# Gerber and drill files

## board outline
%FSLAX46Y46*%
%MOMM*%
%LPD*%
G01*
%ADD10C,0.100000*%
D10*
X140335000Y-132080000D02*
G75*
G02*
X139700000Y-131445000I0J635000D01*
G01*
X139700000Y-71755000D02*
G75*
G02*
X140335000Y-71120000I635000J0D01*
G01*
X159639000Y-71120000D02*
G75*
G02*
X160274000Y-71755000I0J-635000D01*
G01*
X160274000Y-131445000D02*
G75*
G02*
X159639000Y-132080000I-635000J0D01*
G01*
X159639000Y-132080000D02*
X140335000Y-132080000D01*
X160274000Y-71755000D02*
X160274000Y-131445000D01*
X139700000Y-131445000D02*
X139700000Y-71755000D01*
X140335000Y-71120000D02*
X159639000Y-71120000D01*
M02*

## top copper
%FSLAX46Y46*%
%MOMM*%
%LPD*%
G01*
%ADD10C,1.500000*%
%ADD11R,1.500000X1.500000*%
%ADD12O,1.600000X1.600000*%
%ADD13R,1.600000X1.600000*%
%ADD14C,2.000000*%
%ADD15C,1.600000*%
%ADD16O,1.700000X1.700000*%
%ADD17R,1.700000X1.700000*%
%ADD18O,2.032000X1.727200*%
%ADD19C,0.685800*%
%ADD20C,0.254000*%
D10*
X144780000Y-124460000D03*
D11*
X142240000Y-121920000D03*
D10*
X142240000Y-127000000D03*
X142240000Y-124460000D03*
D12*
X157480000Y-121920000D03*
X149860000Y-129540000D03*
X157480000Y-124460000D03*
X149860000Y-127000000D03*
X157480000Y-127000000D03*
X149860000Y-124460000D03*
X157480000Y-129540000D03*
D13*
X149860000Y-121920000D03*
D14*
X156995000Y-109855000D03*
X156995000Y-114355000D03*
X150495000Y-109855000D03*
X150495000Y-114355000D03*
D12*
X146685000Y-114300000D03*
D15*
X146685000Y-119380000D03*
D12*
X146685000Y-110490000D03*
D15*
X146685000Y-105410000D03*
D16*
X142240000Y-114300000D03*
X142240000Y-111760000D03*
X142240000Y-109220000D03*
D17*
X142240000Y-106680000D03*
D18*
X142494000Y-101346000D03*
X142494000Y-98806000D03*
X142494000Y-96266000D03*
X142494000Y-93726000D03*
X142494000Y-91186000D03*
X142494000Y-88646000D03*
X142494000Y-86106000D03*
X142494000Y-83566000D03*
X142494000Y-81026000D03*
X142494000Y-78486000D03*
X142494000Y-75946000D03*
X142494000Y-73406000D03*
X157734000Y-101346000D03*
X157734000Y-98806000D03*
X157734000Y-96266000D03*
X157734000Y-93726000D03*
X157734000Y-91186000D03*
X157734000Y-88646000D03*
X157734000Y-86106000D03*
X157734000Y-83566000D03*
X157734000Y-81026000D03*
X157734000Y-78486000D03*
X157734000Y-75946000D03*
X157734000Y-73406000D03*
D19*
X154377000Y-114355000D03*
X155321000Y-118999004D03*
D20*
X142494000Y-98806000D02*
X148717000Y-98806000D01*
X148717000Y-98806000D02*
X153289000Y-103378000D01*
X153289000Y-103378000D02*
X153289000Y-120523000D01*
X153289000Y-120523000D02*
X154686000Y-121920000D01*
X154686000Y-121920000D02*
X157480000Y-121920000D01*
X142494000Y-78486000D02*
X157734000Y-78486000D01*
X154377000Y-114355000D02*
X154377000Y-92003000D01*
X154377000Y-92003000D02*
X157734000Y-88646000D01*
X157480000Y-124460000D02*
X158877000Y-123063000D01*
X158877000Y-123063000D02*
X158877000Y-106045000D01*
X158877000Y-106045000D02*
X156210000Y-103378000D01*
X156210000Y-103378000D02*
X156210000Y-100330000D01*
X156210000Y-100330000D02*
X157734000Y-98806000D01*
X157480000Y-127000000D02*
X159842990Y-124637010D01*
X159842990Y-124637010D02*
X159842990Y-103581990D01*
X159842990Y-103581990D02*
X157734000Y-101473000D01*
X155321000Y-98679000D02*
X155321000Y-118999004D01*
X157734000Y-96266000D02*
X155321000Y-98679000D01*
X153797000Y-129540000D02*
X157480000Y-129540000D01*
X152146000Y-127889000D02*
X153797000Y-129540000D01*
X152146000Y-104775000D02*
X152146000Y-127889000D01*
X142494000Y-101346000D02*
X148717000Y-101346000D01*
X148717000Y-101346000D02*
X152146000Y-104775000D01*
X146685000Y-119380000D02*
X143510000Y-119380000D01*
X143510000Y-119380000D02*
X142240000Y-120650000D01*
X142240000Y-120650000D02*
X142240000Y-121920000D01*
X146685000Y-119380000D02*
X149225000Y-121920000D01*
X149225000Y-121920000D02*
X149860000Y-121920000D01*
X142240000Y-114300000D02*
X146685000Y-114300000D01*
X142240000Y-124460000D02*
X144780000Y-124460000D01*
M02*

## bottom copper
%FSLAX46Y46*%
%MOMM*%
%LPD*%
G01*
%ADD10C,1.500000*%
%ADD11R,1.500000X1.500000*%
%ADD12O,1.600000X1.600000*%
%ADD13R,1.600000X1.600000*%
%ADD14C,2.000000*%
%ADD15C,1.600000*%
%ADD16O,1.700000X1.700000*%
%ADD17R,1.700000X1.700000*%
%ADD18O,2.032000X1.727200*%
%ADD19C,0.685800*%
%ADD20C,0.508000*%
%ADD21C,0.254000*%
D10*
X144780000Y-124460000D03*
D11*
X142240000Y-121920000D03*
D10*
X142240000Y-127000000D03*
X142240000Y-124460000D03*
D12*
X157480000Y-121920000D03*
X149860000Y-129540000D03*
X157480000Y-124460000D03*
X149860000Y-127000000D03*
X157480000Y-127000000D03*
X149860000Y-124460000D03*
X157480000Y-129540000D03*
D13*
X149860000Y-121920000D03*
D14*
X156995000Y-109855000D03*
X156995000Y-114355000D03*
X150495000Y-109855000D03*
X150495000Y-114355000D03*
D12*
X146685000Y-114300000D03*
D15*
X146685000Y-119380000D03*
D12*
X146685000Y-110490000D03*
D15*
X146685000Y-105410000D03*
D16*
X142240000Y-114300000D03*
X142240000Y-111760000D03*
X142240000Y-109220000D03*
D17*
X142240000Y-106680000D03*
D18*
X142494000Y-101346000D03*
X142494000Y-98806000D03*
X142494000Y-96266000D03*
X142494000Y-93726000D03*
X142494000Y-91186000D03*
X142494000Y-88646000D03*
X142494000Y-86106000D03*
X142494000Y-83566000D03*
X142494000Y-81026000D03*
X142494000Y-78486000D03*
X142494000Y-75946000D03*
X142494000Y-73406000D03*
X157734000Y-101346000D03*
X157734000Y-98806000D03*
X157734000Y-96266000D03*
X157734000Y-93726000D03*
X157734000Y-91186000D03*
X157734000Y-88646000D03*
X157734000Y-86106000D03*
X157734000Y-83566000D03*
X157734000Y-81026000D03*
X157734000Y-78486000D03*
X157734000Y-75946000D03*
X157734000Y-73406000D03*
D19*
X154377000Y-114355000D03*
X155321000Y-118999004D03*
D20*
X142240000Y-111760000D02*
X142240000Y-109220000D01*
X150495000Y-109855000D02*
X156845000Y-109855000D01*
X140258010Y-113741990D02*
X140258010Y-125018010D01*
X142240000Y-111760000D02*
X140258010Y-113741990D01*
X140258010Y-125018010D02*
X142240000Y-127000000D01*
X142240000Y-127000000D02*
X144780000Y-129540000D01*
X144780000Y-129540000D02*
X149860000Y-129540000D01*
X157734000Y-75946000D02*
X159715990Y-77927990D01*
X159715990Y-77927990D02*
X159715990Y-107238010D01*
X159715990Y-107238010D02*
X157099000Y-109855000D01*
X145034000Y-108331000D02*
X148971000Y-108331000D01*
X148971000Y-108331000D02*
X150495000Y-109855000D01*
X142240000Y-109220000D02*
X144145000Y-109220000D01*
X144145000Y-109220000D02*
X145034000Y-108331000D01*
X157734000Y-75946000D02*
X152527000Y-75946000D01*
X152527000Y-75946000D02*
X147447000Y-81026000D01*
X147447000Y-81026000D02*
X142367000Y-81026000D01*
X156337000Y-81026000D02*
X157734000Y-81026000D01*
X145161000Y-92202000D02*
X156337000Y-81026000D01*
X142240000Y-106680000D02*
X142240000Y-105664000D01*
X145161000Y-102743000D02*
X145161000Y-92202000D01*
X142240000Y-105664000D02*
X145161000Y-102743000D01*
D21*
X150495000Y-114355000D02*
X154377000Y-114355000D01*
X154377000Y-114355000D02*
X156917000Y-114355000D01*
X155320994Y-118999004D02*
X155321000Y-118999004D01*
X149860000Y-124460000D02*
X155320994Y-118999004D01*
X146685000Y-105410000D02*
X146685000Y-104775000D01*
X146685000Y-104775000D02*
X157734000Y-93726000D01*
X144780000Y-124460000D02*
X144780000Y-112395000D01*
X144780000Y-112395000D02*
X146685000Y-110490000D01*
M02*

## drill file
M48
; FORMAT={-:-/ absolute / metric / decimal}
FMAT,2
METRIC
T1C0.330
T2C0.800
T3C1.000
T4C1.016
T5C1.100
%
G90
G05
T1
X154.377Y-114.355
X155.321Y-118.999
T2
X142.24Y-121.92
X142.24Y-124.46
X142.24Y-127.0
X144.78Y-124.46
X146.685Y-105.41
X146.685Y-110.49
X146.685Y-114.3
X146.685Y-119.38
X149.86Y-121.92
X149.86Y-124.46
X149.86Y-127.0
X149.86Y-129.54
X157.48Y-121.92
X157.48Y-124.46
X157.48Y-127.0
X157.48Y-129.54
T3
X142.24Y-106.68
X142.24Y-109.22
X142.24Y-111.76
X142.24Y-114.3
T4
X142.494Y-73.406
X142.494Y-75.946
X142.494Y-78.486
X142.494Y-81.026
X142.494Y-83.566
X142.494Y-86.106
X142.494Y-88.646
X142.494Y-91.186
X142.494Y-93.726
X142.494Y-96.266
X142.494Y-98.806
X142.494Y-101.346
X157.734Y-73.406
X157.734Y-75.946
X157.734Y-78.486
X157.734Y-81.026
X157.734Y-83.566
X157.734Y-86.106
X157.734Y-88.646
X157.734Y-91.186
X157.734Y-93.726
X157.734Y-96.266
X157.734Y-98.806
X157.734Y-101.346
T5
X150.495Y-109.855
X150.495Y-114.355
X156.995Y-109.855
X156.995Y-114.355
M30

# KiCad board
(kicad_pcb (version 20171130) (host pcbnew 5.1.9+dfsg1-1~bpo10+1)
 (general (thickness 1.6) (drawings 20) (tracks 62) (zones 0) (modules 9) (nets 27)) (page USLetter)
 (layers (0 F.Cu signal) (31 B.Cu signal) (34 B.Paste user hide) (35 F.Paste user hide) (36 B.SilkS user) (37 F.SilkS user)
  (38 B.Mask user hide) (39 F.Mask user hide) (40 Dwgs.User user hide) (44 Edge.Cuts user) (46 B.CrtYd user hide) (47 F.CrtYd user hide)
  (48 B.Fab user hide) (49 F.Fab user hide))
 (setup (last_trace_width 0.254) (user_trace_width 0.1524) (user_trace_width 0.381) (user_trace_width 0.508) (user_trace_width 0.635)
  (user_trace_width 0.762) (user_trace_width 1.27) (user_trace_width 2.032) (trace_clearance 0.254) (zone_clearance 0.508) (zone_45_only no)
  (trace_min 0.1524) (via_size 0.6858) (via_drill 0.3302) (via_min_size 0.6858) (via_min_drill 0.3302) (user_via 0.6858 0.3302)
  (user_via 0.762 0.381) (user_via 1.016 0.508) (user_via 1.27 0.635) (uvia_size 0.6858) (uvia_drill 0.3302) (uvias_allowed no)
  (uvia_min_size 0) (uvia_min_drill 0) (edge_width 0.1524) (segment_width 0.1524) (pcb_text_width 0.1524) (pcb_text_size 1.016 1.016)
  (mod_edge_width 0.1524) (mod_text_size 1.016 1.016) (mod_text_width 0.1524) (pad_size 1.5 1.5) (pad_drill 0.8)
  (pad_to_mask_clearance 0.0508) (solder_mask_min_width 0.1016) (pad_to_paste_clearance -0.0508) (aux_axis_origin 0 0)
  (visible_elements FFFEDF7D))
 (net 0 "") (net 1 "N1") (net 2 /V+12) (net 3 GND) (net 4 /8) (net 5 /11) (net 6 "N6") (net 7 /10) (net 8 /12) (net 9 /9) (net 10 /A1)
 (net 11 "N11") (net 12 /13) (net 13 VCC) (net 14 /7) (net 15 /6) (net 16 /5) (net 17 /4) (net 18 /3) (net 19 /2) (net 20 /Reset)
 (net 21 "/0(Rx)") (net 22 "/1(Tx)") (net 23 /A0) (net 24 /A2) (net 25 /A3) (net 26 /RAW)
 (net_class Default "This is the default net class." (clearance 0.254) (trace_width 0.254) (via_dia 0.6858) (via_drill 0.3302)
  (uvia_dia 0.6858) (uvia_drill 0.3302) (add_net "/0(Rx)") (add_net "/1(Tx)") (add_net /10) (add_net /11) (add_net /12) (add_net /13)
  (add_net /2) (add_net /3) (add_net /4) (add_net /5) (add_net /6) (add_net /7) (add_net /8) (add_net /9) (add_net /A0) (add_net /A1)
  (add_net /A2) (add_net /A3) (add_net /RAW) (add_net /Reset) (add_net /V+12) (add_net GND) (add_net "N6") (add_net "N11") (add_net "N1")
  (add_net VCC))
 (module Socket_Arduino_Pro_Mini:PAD (layer F.Cu) (at 144.78 124.46)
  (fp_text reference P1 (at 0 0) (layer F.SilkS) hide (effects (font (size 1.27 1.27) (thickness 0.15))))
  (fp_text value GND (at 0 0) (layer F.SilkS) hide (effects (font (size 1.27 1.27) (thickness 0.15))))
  (pad 1 thru_hole circle (at 0 0) (size 1.5 1.5) (drill 0.8) (layers *.Cu *.Mask) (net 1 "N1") (solder_mask_margin 0.0762)))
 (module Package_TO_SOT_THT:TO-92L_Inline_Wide (layer F.Cu) (at 142.24 121.92 270)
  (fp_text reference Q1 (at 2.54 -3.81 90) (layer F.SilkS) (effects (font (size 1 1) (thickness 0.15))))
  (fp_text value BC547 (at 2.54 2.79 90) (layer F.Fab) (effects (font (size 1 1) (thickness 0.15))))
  (pad 1 thru_hole rect (at 0 0 270) (size 1.5 1.5) (drill 0.8) (layers *.Cu *.Mask) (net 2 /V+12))
  (pad 3 thru_hole circle (at 5.08 0 270) (size 1.5 1.5) (drill 0.8) (layers *.Cu *.Mask) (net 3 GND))
  (pad 2 thru_hole circle (at 2.54 0 270) (size 1.5 1.5) (drill 0.8) (layers *.Cu *.Mask) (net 1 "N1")))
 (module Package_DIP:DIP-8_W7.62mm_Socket (layer F.Cu) (at 149.86 121.92)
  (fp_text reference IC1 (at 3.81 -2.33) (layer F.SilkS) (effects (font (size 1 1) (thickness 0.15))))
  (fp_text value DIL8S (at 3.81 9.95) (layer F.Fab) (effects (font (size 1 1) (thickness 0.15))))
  (pad 8 thru_hole oval (at 7.62 0) (size 1.6 1.6) (drill 0.8) (layers *.Cu *.Mask) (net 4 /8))
  (pad 4 thru_hole oval (at 0 7.62) (size 1.6 1.6) (drill 0.8) (layers *.Cu *.Mask) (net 3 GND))
  (pad 7 thru_hole oval (at 7.62 2.54) (size 1.6 1.6) (drill 0.8) (layers *.Cu *.Mask) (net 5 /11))
  (pad 3 thru_hole oval (at 0 5.08) (size 1.6 1.6) (drill 0.8) (layers *.Cu *.Mask) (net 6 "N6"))
  (pad 6 thru_hole oval (at 7.62 5.08) (size 1.6 1.6) (drill 0.8) (layers *.Cu *.Mask) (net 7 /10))
  (pad 2 thru_hole oval (at 0 2.54) (size 1.6 1.6) (drill 0.8) (layers *.Cu *.Mask) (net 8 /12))
  (pad 5 thru_hole oval (at 7.62 7.62) (size 1.6 1.6) (drill 0.8) (layers *.Cu *.Mask) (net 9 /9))
  (pad 1 thru_hole rect (at 0 0) (size 1.6 1.6) (drill 0.8) (layers *.Cu *.Mask) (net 2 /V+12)))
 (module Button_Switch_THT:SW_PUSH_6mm (layer F.Cu) (at 150.495 109.855)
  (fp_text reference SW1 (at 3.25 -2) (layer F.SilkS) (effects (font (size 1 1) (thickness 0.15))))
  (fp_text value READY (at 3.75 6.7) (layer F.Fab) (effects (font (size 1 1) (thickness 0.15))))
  (pad 1 thru_hole circle (at 6.5 0 90) (size 2 2) (drill 1.1) (layers *.Cu *.Mask) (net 3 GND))
  (pad 2 thru_hole circle (at 6.5 4.5 90) (size 2 2) (drill 1.1) (layers *.Cu *.Mask) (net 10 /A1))
  (pad 1 thru_hole circle (at 0 0 90) (size 2 2) (drill 1.1) (layers *.Cu *.Mask) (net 3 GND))
  (pad 2 thru_hole circle (at 0 4.5 90) (size 2 2) (drill 1.1) (layers *.Cu *.Mask) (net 10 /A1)))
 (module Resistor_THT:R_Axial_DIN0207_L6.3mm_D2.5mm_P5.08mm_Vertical (layer F.Cu) (at 146.685 119.38 90)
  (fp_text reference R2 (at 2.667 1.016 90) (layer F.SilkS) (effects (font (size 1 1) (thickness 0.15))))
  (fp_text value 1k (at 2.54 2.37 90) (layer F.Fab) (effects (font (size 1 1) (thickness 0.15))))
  (pad 2 thru_hole oval (at 5.08 0 90) (size 1.6 1.6) (drill 0.8) (layers *.Cu *.Mask) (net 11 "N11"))
  (pad 1 thru_hole circle (at 0 0 90) (size 1.6 1.6) (drill 0.8) (layers *.Cu *.Mask) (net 2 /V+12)))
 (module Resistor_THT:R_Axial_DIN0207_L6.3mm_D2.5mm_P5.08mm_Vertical (layer F.Cu) (at 146.685 105.41 270)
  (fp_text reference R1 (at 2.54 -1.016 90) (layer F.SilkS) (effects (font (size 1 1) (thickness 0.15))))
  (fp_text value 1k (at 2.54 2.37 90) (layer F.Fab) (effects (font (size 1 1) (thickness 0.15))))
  (pad 2 thru_hole oval (at 5.08 0 270) (size 1.6 1.6) (drill 0.8) (layers *.Cu *.Mask) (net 1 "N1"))
  (pad 1 thru_hole circle (at 0 0 270) (size 1.6 1.6) (drill 0.8) (layers *.Cu *.Mask) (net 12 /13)))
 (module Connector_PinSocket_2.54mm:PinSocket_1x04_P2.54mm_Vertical (layer F.Cu) (at 142.24 106.68)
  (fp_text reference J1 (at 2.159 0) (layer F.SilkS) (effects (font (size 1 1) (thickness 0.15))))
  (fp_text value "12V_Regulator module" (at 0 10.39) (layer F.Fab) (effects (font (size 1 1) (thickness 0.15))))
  (pad 4 thru_hole oval (at 0 7.62) (size 1.7 1.7) (drill 1) (layers *.Cu *.Mask) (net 11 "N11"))
  (pad 3 thru_hole oval (at 0 5.08) (size 1.7 1.7) (drill 1) (layers *.Cu *.Mask) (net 3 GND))
  (pad 2 thru_hole oval (at 0 2.54) (size 1.7 1.7) (drill 1) (layers *.Cu *.Mask) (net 3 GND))
  (pad 1 thru_hole rect (at 0 0) (size 1.7 1.7) (drill 1) (layers *.Cu *.Mask) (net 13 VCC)))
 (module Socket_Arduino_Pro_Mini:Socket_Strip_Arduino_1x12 (layer F.Cu) (at 142.494 73.406 270)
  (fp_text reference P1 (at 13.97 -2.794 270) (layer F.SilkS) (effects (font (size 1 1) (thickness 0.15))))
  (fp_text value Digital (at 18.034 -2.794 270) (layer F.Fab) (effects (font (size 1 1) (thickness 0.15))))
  (pad 12 thru_hole oval (at 27.94 0 270) (size 1.7272 2.032) (drill 1.016) (layers *.Cu *.Mask F.SilkS) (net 9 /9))
  (pad 11 thru_hole oval (at 25.4 0 270) (size 1.7272 2.032) (drill 1.016) (layers *.Cu *.Mask F.SilkS) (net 4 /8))
  (pad 10 thru_hole oval (at 22.86 0 270) (size 1.7272 2.032) (drill 1.016) (layers *.Cu *.Mask F.SilkS) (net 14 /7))
  (pad 9 thru_hole oval (at 20.32 0 270) (size 1.7272 2.032) (drill 1.016) (layers *.Cu *.Mask F.SilkS) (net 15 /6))
  (pad 8 thru_hole oval (at 17.78 0 270) (size 1.7272 2.032) (drill 1.016) (layers *.Cu *.Mask F.SilkS) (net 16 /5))
  (pad 7 thru_hole oval (at 15.24 0 270) (size 1.7272 2.032) (drill 1.016) (layers *.Cu *.Mask F.SilkS) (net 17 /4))
  (pad 6 thru_hole oval (at 12.7 0 270) (size 1.7272 2.032) (drill 1.016) (layers *.Cu *.Mask F.SilkS) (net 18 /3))
  (pad 5 thru_hole oval (at 10.16 0 270) (size 1.7272 2.032) (drill 1.016) (layers *.Cu *.Mask F.SilkS) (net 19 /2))
  (pad 4 thru_hole oval (at 7.62 0 270) (size 1.7272 2.032) (drill 1.016) (layers *.Cu *.Mask F.SilkS) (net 3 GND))
  (pad 3 thru_hole oval (at 5.08 0 270) (size 1.7272 2.032) (drill 1.016) (layers *.Cu *.Mask F.SilkS) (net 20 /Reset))
  (pad 2 thru_hole oval (at 2.54 0 270) (size 1.7272 2.032) (drill 1.016) (layers *.Cu *.Mask F.SilkS) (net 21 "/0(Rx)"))
  (pad 1 thru_hole oval (at 0 0 270) (size 1.7272 2.032) (drill 1.016) (layers *.Cu *.Mask F.SilkS) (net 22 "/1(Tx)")))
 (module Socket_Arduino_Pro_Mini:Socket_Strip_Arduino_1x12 (layer F.Cu) (at 157.734 73.406 270)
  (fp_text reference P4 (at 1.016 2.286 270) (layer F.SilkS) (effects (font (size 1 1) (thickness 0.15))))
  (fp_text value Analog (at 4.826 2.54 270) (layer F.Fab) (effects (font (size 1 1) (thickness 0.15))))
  (pad 12 thru_hole oval (at 27.94 0 270) (size 1.7272 2.032) (drill 1.016) (layers *.Cu *.Mask F.SilkS) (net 7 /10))
  (pad 11 thru_hole oval (at 25.4 0 270) (size 1.7272 2.032) (drill 1.016) (layers *.Cu *.Mask F.SilkS) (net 5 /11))
  (pad 10 thru_hole oval (at 22.86 0 270) (size 1.7272 2.032) (drill 1.016) (layers *.Cu *.Mask F.SilkS) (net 8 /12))
  (pad 9 thru_hole oval (at 20.32 0 270) (size 1.7272 2.032) (drill 1.016) (layers *.Cu *.Mask F.SilkS) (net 12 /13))
  (pad 8 thru_hole oval (at 17.78 0 270) (size 1.7272 2.032) (drill 1.016) (layers *.Cu *.Mask F.SilkS) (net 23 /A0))
  (pad 7 thru_hole oval (at 15.24 0 270) (size 1.7272 2.032) (drill 1.016) (layers *.Cu *.Mask F.SilkS) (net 10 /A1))
  (pad 6 thru_hole oval (at 12.7 0 270) (size 1.7272 2.032) (drill 1.016) (layers *.Cu *.Mask F.SilkS) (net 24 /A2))
  (pad 5 thru_hole oval (at 10.16 0 270) (size 1.7272 2.032) (drill 1.016) (layers *.Cu *.Mask F.SilkS) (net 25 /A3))
  (pad 4 thru_hole oval (at 7.62 0 270) (size 1.7272 2.032) (drill 1.016) (layers *.Cu *.Mask F.SilkS) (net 13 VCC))
  (pad 3 thru_hole oval (at 5.08 0 270) (size 1.7272 2.032) (drill 1.016) (layers *.Cu *.Mask F.SilkS) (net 20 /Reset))
  (pad 2 thru_hole oval (at 2.54 0 270) (size 1.7272 2.032) (drill 1.016) (layers *.Cu *.Mask F.SilkS) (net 3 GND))
  (pad 1 thru_hole oval (at 0 0 270) (size 1.7272 2.032) (drill 1.016) (layers *.Cu *.Mask F.SilkS) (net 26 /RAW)))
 (gr_arc (start 140.335 131.445) (end 139.7 131.445) (angle -90) (layer Edge.Cuts) (width 0.1))
 (gr_arc (start 140.335 71.755) (end 140.335 71.12) (angle -90) (layer Edge.Cuts) (width 0.1))
 (gr_arc (start 159.639 71.755) (end 160.274 71.755) (angle -90) (layer Edge.Cuts) (width 0.1))
 (gr_arc (start 159.639 131.445) (end 159.639 132.08) (angle -90) (layer Edge.Cuts) (width 0.1))
 (gr_line (start 159.639 132.08) (end 140.335 132.08) (angle 90) (layer Edge.Cuts) (width 0.1))
 (gr_line (start 160.274 71.755) (end 160.274 131.445) (angle 90) (layer Edge.Cuts) (width 0.1))
 (gr_line (start 139.7 131.445) (end 139.7 71.755) (angle 90) (layer Edge.Cuts) (width 0.1))
 (gr_line (start 140.335 71.12) (end 159.639 71.12) (angle 90) (layer Edge.Cuts) (width 0.1))
 (segment (start 142.494 98.806) (end 148.717 98.806) (width 0.254) (layer F.Cu) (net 4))
 (segment (start 148.717 98.806) (end 153.289 103.378) (width 0.254) (layer F.Cu) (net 4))
 (segment (start 153.289 103.378) (end 153.289 120.523) (width 0.254) (layer F.Cu) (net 4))
 (segment (start 153.289 120.523) (end 154.686 121.92) (width 0.254) (layer F.Cu) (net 4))
 (segment (start 154.686 121.92) (end 157.48 121.92) (width 0.254) (layer F.Cu) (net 4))
 (segment (start 142.24 111.76) (end 142.24 109.22) (width 0.508) (layer B.Cu) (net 3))
 (segment (start 150.495 109.855) (end 156.845 109.855) (width 0.508) (layer B.Cu) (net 3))
 (segment (start 140.25801 113.74199) (end 140.25801 125.01801) (width 0.508) (layer B.Cu) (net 3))
 (segment (start 142.24 111.76) (end 140.25801 113.74199) (width 0.508) (layer B.Cu) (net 3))
 (segment (start 140.25801 125.01801) (end 142.24 127) (width 0.508) (layer B.Cu) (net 3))
 (segment (start 142.24 127) (end 144.78 129.54) (width 0.508) (layer B.Cu) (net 3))
 (segment (start 144.78 129.54) (end 149.86 129.54) (width 0.508) (layer B.Cu) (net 3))
 (segment (start 157.734 75.946) (end 159.71599 77.92799) (width 0.508) (layer B.Cu) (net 3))
 (segment (start 159.71599 77.92799) (end 159.71599 107.23801) (width 0.508) (layer B.Cu) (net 3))
 (segment (start 159.71599 107.23801) (end 157.099 109.855) (width 0.508) (layer B.Cu) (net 3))
 (segment (start 145.034 108.331) (end 148.971 108.331) (width 0.508) (layer B.Cu) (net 3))
 (segment (start 148.971 108.331) (end 150.495 109.855) (width 0.508) (layer B.Cu) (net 3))
 (segment (start 142.24 109.22) (end 144.145 109.22) (width 0.508) (layer B.Cu) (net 3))
 (segment (start 144.145 109.22) (end 145.034 108.331) (width 0.508) (layer B.Cu) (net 3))
 (segment (start 157.734 75.946) (end 152.527 75.946) (width 0.508) (layer B.Cu) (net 3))
 (segment (start 152.527 75.946) (end 147.447 81.026) (width 0.508) (layer B.Cu) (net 3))
 (segment (start 147.447 81.026) (end 142.367 81.026) (width 0.508) (layer B.Cu) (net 3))
 (segment (start 142.494 78.486) (end 157.734 78.486) (width 0.254) (layer F.Cu) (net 20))
 (segment (start 156.337 81.026) (end 157.734 81.026) (width 0.508) (layer B.Cu) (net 13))
 (segment (start 145.161 92.202) (end 156.337 81.026) (width 0.508) (layer B.Cu) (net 13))
 (segment (start 142.24 106.68) (end 142.24 105.664) (width 0.508) (layer B.Cu) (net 13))
 (segment (start 145.161 102.743) (end 145.161 92.202) (width 0.508) (layer B.Cu) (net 13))
 (segment (start 142.24 105.664) (end 145.161 102.743) (width 0.508) (layer B.Cu) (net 13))
 (segment (start 150.495 114.355) (end 154.377 114.355) (width 0.254) (layer B.Cu) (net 10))
 (segment (start 154.377 114.355) (end 156.917 114.355) (width 0.254) (layer B.Cu) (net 10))
 (via (at 154.377 114.355) (size 0.6858) (drill 0.3302) (layers F.Cu B.Cu) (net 10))
 (segment (start 154.377 114.355) (end 154.377 92.003) (width 0.254) (layer F.Cu) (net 10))
 (segment (start 154.377 92.003) (end 157.734 88.646) (width 0.254) (layer F.Cu) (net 10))
 (segment (start 157.48 124.46) (end 158.877 123.063) (width 0.254) (layer F.Cu) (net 5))
 (segment (start 158.877 123.063) (end 158.877 106.045) (width 0.254) (layer F.Cu) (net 5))
 (segment (start 158.877 106.045) (end 156.21 103.378) (width 0.254) (layer F.Cu) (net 5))
 (segment (start 156.21 103.378) (end 156.21 100.33) (width 0.254) (layer F.Cu) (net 5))
 (segment (start 156.21 100.33) (end 157.734 98.806) (width 0.254) (layer F.Cu) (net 5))
 (segment (start 157.48 127) (end 159.84299 124.63701) (width 0.254) (layer F.Cu) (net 7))
 (segment (start 159.84299 124.63701) (end 159.84299 103.58199) (width 0.254) (layer F.Cu) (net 7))
 (segment (start 159.84299 103.58199) (end 157.734 101.473) (width 0.254) (layer F.Cu) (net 7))
 (via (at 155.321 118.999004) (size 0.6858) (drill 0.3302) (layers F.Cu B.Cu) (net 8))
 (segment (start 155.320994 118.999004) (end 155.321 118.999004) (width 0.254) (layer B.Cu) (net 8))
 (segment (start 149.86 124.46) (end 155.320994 118.999004) (width 0.254) (layer B.Cu) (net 8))
 (segment (start 155.321 98.679) (end 155.321 118.999004) (width 0.254) (layer F.Cu) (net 8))
 (segment (start 157.734 96.266) (end 155.321 98.679) (width 0.254) (layer F.Cu) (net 8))
 (segment (start 153.797 129.54) (end 157.48 129.54) (width 0.254) (layer F.Cu) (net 9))
 (segment (start 152.146 127.889) (end 153.797 129.54) (width 0.254) (layer F.Cu) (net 9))
 (segment (start 152.146 104.775) (end 152.146 127.889) (width 0.254) (layer F.Cu) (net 9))
 (segment (start 142.494 101.346) (end 148.717 101.346) (width 0.254) (layer F.Cu) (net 9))
 (segment (start 148.717 101.346) (end 152.146 104.775) (width 0.254) (layer F.Cu) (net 9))
 (segment (start 146.685 119.38) (end 143.51 119.38) (width 0.254) (layer F.Cu) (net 2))
 (segment (start 143.51 119.38) (end 142.24 120.65) (width 0.254) (layer F.Cu) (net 2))
 (segment (start 142.24 120.65) (end 142.24 121.92) (width 0.254) (layer F.Cu) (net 2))
 (segment (start 146.685 119.38) (end 149.225 121.92) (width 0.254) (layer F.Cu) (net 2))
 (segment (start 149.225 121.92) (end 149.86 121.92) (width 0.254) (layer F.Cu) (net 2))
 (segment (start 142.24 114.3) (end 146.685 114.3) (width 0.254) (layer F.Cu) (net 11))
 (segment (start 146.685 105.41) (end 146.685 104.775) (width 0.254) (layer B.Cu) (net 12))
 (segment (start 146.685 104.775) (end 157.734 93.726) (width 0.254) (layer B.Cu) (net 12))
 (segment (start 142.24 124.46) (end 144.78 124.46) (width 0.254) (layer F.Cu) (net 1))
 (segment (start 144.78 124.46) (end 144.78 112.395) (width 0.254) (layer B.Cu) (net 1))
 (segment (start 144.78 112.395) (end 146.685 110.49) (width 0.254) (layer B.Cu) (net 1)))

